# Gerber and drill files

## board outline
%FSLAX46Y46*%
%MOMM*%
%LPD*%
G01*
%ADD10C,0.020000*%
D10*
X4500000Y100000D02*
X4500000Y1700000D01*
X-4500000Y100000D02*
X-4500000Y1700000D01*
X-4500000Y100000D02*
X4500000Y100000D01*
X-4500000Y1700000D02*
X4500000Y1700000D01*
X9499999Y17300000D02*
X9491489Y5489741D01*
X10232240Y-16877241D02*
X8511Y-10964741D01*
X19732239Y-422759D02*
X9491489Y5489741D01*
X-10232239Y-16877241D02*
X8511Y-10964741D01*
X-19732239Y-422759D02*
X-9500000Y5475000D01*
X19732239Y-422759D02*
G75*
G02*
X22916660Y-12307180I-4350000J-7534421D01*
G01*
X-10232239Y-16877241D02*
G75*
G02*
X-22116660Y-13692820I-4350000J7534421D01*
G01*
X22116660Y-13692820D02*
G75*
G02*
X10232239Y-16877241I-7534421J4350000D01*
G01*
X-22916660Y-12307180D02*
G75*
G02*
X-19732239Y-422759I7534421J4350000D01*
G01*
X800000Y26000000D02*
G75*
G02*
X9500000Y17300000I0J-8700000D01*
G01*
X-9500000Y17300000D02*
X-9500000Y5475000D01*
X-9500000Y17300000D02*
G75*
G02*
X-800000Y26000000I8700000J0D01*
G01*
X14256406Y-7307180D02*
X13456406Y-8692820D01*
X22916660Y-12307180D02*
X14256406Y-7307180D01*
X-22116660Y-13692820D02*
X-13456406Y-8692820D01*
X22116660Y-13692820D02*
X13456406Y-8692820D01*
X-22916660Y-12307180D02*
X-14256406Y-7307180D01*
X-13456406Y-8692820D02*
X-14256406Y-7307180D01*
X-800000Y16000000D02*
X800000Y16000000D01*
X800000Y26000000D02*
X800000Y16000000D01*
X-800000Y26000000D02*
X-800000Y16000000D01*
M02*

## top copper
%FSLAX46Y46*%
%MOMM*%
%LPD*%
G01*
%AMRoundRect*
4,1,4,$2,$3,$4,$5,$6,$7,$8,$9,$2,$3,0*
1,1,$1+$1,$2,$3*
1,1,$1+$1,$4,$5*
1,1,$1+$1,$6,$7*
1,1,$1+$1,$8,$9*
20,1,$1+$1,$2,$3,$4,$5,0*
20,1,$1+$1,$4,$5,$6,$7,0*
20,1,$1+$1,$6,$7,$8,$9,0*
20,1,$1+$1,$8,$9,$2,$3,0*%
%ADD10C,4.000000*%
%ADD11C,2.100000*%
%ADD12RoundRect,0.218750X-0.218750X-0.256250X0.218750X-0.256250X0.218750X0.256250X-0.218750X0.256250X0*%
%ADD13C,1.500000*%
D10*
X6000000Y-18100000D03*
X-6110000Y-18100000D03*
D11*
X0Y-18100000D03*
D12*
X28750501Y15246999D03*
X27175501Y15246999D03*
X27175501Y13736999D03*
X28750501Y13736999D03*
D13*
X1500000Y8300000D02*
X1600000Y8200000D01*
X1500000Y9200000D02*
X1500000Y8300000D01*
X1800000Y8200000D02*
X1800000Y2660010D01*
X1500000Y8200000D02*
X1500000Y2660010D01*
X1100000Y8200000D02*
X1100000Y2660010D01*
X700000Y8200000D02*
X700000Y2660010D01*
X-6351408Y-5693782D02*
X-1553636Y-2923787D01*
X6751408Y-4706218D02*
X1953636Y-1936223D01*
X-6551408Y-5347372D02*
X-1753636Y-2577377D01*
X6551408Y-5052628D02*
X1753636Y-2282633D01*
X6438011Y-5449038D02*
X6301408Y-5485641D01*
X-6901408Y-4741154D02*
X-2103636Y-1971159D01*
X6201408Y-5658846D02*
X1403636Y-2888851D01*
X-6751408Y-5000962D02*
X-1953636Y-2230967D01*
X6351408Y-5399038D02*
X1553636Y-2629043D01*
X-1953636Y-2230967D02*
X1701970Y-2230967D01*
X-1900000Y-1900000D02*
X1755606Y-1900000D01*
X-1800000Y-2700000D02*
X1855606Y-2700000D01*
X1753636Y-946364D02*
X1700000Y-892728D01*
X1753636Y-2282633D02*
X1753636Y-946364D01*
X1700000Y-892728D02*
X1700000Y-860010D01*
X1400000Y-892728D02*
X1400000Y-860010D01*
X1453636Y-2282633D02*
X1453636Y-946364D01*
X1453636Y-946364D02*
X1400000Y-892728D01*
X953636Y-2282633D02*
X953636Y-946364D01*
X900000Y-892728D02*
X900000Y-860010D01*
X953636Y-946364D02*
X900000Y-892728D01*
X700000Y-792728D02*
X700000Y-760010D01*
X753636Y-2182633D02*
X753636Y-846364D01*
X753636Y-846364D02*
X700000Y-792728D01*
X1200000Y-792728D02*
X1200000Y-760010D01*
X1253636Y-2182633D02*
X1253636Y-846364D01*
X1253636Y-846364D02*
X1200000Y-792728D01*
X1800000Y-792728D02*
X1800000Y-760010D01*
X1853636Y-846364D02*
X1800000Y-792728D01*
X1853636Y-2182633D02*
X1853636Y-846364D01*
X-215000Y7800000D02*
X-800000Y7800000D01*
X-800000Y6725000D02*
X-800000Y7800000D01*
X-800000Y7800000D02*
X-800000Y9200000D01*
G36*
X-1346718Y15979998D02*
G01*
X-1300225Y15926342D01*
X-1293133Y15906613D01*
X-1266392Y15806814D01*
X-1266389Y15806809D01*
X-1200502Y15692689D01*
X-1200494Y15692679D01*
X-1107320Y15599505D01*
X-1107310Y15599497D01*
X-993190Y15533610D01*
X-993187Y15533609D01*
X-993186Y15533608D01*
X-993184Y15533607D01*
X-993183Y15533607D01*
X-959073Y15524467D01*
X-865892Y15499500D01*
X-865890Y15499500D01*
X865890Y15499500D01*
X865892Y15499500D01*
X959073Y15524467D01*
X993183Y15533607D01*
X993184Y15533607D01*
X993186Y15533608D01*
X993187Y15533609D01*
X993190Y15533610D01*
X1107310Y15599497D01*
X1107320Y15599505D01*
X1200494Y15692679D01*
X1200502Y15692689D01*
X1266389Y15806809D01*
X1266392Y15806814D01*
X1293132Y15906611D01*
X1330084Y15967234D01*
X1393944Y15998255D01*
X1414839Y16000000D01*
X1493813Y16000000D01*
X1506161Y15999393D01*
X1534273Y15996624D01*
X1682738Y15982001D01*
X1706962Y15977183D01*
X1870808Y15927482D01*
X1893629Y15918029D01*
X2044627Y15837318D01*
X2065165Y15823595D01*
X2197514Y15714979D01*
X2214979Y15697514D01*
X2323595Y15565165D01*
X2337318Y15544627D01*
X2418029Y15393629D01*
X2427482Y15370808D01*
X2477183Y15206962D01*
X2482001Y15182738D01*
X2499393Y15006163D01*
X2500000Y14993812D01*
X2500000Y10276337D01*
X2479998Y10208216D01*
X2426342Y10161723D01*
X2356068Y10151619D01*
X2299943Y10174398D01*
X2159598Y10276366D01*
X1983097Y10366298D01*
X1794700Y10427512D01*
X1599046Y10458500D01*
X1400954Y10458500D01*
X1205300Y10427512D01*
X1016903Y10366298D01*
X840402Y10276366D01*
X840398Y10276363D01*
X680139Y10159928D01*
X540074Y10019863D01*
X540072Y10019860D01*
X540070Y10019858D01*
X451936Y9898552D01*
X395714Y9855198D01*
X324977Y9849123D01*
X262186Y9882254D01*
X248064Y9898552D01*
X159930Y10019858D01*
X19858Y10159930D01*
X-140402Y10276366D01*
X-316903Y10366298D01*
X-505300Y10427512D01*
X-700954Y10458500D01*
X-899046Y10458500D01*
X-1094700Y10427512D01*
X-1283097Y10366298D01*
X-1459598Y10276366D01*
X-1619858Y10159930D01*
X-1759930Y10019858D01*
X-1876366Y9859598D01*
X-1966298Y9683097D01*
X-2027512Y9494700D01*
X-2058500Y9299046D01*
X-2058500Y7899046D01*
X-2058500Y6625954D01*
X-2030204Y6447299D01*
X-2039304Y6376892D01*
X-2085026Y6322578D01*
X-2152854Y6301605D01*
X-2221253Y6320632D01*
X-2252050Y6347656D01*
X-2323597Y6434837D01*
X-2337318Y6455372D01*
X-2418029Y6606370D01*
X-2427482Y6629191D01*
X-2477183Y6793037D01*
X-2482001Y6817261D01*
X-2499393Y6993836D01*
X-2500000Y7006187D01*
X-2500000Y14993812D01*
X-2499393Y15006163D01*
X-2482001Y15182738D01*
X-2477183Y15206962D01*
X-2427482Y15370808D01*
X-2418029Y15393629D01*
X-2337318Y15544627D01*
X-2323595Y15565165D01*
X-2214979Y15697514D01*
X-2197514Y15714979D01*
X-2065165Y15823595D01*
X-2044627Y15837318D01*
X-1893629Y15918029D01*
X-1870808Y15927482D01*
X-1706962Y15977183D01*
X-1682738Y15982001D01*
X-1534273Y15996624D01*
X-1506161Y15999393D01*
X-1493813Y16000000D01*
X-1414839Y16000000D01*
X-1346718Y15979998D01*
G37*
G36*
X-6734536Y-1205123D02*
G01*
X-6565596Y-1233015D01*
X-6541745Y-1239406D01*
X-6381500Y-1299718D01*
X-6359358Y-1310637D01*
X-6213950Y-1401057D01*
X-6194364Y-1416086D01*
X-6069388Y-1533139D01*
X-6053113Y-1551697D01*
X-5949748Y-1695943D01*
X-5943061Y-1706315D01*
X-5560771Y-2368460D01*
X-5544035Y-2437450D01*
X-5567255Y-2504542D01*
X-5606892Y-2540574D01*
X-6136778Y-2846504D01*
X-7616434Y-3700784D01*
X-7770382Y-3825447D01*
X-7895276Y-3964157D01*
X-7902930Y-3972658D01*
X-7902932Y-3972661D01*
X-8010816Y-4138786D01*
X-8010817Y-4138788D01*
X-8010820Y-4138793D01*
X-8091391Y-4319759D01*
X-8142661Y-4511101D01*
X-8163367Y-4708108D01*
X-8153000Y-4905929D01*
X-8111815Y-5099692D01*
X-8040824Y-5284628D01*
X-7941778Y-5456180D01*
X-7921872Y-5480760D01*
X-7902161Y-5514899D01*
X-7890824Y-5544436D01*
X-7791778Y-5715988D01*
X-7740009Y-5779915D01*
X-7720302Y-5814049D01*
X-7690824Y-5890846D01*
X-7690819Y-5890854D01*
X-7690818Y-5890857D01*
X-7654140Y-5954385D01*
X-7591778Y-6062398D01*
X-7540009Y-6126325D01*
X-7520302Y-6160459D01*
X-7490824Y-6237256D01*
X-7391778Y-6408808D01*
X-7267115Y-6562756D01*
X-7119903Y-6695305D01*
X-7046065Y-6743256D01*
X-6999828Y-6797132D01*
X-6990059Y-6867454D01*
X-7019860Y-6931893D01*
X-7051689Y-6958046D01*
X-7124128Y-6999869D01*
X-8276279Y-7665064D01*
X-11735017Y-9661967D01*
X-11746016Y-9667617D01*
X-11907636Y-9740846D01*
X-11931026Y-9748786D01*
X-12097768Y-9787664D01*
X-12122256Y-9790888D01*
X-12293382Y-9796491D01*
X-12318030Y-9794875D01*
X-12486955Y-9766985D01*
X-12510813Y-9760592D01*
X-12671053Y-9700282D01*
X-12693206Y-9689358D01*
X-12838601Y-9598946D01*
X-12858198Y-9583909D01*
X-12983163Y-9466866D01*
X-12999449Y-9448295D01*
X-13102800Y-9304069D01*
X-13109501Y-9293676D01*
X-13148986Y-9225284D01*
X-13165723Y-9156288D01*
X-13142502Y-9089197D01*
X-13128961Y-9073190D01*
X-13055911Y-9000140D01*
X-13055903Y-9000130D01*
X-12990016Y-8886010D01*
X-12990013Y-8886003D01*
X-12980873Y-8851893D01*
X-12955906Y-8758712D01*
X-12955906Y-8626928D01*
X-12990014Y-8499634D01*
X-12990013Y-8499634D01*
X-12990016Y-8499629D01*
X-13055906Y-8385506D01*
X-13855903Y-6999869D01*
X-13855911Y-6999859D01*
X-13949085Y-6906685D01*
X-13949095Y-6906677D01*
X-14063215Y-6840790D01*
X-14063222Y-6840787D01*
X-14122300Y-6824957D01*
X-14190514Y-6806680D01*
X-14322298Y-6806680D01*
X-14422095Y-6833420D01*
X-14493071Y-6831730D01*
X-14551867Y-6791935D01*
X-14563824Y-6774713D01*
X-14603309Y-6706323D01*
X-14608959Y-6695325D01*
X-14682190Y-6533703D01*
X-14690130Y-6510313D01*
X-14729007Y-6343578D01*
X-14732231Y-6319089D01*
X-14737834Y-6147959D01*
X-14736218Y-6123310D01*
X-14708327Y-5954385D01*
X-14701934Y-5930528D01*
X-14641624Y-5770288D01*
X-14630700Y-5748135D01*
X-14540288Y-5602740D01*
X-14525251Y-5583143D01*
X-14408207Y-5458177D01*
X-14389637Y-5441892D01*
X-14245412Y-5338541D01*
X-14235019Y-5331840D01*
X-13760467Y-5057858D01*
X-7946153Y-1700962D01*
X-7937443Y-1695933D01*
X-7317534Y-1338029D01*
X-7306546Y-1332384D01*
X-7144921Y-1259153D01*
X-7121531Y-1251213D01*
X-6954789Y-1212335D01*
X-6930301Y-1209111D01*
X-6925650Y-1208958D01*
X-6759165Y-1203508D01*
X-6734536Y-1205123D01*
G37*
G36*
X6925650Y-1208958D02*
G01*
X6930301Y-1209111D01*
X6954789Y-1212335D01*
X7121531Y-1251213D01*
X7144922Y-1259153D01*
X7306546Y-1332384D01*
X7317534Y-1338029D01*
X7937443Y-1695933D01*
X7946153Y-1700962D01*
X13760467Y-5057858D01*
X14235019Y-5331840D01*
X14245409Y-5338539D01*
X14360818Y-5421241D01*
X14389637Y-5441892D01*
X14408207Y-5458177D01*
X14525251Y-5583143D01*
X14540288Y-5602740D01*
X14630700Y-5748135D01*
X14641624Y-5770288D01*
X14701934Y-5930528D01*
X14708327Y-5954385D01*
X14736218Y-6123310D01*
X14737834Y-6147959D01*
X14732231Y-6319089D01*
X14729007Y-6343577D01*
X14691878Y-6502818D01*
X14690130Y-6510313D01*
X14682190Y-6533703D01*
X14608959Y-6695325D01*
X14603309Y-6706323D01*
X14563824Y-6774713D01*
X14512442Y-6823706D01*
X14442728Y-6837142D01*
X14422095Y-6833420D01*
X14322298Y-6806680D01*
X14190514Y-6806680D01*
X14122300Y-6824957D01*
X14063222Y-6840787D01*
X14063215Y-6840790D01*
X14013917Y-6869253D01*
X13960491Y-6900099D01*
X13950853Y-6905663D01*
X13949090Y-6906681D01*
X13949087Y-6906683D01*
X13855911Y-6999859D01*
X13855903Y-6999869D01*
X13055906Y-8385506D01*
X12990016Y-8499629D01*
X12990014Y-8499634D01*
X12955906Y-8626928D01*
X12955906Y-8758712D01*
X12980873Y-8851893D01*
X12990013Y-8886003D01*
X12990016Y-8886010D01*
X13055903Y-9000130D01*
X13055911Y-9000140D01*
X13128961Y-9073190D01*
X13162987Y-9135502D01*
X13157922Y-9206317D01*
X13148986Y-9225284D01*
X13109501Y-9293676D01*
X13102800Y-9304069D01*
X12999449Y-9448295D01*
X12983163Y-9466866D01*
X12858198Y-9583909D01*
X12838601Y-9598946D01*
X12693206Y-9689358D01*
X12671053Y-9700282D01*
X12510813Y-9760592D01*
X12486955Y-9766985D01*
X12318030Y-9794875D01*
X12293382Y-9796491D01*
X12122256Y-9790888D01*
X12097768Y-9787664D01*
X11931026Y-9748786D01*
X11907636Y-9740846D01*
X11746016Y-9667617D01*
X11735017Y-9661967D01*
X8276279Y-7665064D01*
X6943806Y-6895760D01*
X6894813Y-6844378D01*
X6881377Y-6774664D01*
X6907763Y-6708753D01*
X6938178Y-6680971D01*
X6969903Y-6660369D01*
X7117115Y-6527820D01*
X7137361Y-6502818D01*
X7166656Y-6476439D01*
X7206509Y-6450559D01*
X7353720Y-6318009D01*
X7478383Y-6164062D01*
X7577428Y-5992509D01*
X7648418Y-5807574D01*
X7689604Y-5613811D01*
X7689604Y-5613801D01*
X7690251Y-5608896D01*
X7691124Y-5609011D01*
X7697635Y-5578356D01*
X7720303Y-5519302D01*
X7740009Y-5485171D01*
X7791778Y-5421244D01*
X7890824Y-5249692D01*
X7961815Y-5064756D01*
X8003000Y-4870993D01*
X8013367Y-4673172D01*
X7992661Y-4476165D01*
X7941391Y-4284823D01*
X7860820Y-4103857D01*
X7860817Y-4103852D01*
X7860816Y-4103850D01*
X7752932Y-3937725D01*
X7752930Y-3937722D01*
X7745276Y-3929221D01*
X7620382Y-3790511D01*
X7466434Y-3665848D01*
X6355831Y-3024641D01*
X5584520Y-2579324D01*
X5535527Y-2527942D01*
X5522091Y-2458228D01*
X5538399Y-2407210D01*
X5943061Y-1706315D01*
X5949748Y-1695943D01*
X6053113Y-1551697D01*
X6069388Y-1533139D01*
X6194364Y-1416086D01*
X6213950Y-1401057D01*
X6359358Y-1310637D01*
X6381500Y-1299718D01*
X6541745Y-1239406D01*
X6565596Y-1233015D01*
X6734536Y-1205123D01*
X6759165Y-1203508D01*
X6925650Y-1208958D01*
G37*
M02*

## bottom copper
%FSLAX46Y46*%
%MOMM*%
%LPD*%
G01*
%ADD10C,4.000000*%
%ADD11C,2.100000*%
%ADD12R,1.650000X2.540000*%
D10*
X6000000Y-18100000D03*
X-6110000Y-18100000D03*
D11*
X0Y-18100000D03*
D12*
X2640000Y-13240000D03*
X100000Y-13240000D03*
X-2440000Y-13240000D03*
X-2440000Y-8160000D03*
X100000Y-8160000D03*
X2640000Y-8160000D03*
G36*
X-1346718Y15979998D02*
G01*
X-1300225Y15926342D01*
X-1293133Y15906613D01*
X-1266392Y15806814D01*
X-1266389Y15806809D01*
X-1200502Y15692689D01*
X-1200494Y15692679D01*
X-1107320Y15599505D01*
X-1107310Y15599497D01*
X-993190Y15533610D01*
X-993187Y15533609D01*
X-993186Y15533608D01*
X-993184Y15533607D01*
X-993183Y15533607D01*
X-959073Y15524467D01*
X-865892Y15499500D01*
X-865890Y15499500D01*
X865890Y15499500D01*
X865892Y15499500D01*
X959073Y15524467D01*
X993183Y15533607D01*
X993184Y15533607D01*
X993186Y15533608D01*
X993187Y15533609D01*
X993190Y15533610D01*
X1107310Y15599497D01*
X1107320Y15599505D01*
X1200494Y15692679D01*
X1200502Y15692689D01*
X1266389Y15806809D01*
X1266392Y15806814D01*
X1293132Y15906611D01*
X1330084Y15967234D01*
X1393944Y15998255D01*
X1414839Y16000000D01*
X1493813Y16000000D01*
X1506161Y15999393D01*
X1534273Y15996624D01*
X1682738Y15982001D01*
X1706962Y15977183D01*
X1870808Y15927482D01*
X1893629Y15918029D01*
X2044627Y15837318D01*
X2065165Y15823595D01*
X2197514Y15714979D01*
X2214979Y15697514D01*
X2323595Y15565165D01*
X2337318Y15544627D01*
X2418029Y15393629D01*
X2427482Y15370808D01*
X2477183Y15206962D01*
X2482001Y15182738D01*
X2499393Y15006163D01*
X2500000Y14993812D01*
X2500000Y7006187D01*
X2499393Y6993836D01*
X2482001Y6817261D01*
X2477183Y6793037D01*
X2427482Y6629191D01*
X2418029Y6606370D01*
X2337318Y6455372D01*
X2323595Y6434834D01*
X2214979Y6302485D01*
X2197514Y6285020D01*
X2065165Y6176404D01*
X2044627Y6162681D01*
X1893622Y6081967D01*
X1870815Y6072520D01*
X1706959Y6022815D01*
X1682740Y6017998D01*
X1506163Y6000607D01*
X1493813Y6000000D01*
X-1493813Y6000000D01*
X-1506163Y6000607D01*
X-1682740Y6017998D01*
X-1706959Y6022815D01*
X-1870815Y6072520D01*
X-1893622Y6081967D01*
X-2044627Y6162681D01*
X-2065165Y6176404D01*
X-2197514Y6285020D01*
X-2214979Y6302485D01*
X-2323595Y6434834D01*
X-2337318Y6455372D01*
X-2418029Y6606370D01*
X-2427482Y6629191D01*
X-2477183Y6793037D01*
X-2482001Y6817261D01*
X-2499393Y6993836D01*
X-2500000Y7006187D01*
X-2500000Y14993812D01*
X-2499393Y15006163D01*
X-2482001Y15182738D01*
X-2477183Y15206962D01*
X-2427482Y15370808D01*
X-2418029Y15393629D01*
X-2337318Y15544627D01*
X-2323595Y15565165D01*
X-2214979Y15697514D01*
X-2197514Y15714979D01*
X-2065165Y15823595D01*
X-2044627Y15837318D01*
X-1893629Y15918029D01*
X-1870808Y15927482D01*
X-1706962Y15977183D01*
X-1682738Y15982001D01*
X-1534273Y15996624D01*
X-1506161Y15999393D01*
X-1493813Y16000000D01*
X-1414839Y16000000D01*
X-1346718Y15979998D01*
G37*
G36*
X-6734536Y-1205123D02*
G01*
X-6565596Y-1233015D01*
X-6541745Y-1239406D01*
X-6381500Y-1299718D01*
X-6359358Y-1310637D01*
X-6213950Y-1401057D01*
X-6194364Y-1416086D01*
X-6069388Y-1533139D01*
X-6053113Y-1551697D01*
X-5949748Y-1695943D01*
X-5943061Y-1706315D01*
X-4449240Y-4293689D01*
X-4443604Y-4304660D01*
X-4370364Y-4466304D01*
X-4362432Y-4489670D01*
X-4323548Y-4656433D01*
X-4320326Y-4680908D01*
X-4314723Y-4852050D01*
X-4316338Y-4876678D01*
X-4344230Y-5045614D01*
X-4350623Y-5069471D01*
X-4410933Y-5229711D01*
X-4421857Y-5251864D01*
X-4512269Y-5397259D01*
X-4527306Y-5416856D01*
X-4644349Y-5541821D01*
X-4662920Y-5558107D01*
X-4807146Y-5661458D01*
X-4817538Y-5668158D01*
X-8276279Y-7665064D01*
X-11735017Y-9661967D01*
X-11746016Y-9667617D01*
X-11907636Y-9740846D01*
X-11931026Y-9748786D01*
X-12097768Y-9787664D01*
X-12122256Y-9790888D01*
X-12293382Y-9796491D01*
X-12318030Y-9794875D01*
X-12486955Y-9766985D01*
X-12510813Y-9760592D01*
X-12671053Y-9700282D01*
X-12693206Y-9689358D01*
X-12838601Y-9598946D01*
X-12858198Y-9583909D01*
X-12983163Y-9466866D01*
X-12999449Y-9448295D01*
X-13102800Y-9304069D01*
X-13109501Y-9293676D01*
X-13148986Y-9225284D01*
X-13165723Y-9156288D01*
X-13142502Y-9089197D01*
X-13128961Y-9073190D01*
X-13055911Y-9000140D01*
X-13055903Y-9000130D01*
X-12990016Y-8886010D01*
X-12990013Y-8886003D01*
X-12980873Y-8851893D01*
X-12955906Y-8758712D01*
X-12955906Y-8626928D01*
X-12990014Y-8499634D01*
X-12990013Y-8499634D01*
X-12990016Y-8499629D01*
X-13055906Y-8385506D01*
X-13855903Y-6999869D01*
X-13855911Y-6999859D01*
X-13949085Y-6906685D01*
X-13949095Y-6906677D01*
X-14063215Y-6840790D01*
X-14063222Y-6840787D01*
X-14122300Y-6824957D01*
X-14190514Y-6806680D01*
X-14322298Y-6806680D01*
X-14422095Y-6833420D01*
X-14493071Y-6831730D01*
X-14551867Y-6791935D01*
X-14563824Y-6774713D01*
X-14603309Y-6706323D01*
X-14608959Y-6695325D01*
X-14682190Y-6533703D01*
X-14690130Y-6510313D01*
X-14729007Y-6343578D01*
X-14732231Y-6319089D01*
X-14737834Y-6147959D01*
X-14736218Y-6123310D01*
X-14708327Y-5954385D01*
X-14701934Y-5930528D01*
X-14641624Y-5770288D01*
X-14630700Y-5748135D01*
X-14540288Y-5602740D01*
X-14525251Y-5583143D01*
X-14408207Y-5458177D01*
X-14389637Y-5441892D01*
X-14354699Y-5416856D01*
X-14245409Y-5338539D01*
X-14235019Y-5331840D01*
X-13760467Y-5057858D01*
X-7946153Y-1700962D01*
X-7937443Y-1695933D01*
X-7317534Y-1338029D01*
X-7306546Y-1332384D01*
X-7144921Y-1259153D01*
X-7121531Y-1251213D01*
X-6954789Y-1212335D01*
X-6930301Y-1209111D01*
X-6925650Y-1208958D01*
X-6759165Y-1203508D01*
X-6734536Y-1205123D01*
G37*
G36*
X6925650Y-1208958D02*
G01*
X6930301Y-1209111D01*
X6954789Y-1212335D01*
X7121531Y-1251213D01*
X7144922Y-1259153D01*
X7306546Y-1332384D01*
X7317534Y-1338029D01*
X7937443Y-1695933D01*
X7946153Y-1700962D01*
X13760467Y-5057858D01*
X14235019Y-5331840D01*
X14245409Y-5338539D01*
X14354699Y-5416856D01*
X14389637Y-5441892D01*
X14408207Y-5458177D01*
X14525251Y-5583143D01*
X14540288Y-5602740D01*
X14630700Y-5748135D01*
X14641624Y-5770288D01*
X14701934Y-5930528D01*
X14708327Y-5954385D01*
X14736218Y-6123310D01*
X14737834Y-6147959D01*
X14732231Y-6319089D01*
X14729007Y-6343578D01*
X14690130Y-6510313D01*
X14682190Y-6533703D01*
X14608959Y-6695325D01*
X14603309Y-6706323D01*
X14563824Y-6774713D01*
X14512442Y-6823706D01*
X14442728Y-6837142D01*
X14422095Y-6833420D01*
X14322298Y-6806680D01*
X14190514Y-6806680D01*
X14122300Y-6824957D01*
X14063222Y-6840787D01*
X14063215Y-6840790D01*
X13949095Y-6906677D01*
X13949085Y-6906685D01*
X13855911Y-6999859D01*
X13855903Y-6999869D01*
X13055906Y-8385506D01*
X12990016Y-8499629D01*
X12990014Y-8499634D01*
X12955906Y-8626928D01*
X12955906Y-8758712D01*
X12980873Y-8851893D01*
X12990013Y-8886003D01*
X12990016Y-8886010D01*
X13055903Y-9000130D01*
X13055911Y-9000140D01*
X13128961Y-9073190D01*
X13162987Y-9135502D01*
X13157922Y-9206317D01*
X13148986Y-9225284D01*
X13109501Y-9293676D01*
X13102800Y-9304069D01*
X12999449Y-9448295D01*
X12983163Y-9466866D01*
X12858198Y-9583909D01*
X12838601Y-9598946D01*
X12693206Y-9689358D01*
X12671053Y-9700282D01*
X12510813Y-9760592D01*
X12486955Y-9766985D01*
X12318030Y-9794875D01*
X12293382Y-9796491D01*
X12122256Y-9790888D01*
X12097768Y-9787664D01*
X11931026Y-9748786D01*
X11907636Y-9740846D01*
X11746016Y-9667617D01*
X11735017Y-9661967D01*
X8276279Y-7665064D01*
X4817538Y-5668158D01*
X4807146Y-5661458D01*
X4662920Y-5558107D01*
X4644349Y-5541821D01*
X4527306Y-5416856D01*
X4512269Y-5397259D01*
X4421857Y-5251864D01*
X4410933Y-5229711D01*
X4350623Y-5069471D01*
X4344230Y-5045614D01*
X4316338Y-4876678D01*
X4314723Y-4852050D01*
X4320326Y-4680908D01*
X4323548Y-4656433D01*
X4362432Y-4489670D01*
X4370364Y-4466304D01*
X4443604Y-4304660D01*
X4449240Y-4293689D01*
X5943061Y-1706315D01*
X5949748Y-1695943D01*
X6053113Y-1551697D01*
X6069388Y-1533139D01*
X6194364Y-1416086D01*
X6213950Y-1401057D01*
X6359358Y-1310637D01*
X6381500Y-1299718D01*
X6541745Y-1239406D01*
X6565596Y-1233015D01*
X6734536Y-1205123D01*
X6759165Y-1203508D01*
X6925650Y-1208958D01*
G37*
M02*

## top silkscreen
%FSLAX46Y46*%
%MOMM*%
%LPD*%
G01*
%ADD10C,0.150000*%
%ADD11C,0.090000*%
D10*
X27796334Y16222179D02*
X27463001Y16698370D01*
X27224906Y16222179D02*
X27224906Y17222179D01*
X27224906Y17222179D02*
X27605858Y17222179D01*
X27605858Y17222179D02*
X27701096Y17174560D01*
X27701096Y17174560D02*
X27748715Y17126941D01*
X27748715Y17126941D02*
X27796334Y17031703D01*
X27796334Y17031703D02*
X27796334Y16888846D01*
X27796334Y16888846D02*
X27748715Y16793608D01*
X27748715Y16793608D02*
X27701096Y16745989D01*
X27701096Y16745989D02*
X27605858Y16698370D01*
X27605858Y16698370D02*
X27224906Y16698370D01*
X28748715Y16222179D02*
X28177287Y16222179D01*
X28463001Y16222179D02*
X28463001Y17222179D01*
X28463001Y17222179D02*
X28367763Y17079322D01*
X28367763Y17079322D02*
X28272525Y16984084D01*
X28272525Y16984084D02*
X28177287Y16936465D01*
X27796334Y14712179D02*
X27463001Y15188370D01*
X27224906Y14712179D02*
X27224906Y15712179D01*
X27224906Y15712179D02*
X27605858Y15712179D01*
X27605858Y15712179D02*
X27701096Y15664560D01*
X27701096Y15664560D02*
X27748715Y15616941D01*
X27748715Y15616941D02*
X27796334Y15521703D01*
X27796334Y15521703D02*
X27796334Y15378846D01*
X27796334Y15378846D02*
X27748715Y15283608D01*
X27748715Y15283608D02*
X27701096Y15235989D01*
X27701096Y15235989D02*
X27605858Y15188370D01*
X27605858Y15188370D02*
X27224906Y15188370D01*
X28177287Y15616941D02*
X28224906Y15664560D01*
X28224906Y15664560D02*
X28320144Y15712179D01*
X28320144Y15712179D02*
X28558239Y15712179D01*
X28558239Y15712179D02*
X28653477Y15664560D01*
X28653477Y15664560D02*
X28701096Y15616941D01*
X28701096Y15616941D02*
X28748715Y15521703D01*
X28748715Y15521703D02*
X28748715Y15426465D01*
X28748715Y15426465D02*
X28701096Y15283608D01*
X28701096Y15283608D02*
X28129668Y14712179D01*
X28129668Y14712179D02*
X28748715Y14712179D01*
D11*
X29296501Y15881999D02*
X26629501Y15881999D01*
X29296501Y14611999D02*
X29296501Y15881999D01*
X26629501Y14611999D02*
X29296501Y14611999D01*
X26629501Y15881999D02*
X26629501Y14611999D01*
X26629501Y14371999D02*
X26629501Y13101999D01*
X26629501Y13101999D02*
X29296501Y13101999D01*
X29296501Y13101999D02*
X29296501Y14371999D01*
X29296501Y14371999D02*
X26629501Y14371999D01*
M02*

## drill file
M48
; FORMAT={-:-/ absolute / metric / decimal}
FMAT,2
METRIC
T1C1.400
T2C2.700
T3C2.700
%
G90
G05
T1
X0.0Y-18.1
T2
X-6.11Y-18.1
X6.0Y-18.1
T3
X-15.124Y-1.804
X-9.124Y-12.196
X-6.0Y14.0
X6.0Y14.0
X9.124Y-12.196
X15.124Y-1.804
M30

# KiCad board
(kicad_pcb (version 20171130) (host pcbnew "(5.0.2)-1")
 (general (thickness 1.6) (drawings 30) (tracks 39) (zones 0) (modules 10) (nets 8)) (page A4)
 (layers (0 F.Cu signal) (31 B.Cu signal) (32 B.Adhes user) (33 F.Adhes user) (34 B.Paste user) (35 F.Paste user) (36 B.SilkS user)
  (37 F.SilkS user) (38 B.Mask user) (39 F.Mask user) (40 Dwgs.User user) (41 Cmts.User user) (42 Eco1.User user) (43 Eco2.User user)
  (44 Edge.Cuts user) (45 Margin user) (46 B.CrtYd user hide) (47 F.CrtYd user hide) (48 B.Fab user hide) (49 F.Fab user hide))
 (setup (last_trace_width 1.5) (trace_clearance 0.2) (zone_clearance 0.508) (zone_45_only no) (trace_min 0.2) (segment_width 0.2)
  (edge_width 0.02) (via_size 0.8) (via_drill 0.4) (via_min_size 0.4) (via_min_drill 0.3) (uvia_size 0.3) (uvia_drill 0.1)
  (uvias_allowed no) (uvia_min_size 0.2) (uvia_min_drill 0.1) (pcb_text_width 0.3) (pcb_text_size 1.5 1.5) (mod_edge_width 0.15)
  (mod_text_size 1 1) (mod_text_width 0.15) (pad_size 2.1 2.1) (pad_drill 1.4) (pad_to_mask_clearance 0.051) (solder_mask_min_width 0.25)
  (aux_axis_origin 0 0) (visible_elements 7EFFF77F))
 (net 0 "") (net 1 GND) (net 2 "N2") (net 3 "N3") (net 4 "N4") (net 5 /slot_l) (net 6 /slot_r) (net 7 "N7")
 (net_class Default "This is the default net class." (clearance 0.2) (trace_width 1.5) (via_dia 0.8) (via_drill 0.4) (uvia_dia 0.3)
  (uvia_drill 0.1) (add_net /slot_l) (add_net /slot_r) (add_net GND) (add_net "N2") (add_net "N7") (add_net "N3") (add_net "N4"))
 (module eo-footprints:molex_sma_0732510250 (layer F.Cu) (at 0 18.1 180)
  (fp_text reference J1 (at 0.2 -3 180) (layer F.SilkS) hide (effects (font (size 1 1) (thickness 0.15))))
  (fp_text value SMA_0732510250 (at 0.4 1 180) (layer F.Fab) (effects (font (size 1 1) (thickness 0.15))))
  (pad 2 thru_hole circle (at -6 0 180) (size 4 4) (drill 2.7) (layers *.Cu *.Mask) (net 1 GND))
  (pad 2 thru_hole circle (at 6.11 0 180) (size 4 4) (drill 2.7) (layers *.Cu *.Mask) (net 1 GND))
  (pad 1 thru_hole circle (at 0 0 180) (size 2.1 2.1) (drill 1.4) (layers *.Cu *.Mask) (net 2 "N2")))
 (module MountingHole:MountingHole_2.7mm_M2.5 (layer F.Cu) (at 15.124356 1.803848 240)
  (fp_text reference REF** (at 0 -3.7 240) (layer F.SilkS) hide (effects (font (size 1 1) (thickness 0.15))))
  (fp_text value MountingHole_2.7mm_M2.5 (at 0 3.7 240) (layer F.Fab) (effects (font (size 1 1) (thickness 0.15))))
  (pad 1 np_thru_hole circle (at 0 0 240) (size 2.7 2.7) (drill 2.7) (layers *.Cu *.Mask)))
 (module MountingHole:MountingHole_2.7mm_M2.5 (layer F.Cu) (at -9.124356 12.196152 120)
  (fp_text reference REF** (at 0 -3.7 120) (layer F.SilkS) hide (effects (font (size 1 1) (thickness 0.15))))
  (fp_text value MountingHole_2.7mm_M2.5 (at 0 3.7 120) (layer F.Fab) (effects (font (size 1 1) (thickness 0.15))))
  (pad 1 np_thru_hole circle (at 0 0 120) (size 2.7 2.7) (drill 2.7) (layers *.Cu *.Mask)))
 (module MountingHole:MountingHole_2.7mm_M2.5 (layer F.Cu) (at 9.124356 12.196152 240)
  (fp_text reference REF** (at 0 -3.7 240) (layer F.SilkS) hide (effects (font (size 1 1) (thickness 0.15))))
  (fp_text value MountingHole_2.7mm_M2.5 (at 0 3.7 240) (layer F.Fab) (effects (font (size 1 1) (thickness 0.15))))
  (pad 1 np_thru_hole circle (at 0 0 240) (size 2.7 2.7) (drill 2.7) (layers *.Cu *.Mask)))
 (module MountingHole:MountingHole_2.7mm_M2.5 (layer F.Cu) (at -15.124356 1.803848 120)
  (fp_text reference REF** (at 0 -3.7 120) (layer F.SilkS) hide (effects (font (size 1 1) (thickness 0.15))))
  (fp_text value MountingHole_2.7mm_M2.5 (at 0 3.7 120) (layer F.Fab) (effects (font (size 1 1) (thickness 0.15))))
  (pad 1 np_thru_hole circle (at 0 0 120) (size 2.7 2.7) (drill 2.7) (layers *.Cu *.Mask)))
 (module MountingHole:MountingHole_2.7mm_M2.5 (layer F.Cu) (at 6 -14)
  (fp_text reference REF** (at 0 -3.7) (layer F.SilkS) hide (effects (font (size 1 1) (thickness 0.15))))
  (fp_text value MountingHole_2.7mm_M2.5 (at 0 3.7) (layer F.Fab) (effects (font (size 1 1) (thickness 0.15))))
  (pad 1 np_thru_hole circle (at 0 0) (size 2.7 2.7) (drill 2.7) (layers *.Cu *.Mask)))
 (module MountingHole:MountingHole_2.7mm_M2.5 (layer F.Cu) (at -6 -14)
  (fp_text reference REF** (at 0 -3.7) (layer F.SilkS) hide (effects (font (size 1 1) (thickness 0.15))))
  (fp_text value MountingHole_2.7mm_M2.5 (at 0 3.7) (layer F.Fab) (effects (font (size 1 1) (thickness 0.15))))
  (pad 1 np_thru_hole circle (at 0 0) (size 2.7 2.7) (drill 2.7) (layers *.Cu *.Mask)))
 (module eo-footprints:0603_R (layer F.Cu) (at 27.963001 -15.246999)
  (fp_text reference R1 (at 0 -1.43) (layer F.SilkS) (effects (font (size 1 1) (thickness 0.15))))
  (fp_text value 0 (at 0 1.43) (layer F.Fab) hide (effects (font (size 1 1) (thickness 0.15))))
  (fp_line (start 1.3335 -0.635) (end -1.3335 -0.635) (layer F.SilkS) (width 0.09))
  (fp_line (start 1.3335 0.635) (end 1.3335 -0.635) (layer F.SilkS) (width 0.09))
  (fp_line (start -1.3335 0.635) (end 1.3335 0.635) (layer F.SilkS) (width 0.09))
  (fp_line (start -1.3335 -0.635) (end -1.3335 0.635) (layer F.SilkS) (width 0.09))
  (pad 2 smd roundrect (at 0.7875 0) (size 0.875 0.95) (layers F.Cu F.Paste F.Mask) (roundrect_rratio 0.25) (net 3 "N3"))
  (pad 1 smd roundrect (at -0.7875 0) (size 0.875 0.95) (layers F.Cu F.Paste F.Mask) (roundrect_rratio 0.25) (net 1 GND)))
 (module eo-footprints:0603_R (layer F.Cu) (at 27.963001 -13.736999)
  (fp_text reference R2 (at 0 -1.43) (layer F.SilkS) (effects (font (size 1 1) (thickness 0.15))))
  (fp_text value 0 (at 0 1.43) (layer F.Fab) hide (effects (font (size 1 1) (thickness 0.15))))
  (fp_line (start -1.3335 -0.635) (end -1.3335 0.635) (layer F.SilkS) (width 0.09))
  (fp_line (start -1.3335 0.635) (end 1.3335 0.635) (layer F.SilkS) (width 0.09))
  (fp_line (start 1.3335 0.635) (end 1.3335 -0.635) (layer F.SilkS) (width 0.09))
  (fp_line (start 1.3335 -0.635) (end -1.3335 -0.635) (layer F.SilkS) (width 0.09))
  (pad 1 smd roundrect (at -0.7875 0) (size 0.875 0.95) (layers F.Cu F.Paste F.Mask) (roundrect_rratio 0.25) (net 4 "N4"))
  (pad 2 smd roundrect (at 0.7875 0) (size 0.875 0.95) (layers F.Cu F.Paste F.Mask) (roundrect_rratio 0.25) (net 1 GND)))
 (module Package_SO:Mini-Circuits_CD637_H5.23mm (layer B.Cu) (at 0.1 10.7 90)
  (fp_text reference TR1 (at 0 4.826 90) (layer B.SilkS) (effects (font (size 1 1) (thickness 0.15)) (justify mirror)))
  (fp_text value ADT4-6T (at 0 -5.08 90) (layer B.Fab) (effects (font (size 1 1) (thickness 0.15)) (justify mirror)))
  (pad 1 smd rect (at -2.54 2.54 90) (size 2.54 1.65) (layers B.Cu B.Paste B.Mask) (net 4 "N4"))
  (pad 2 smd rect (at -2.54 0 90) (size 2.54 1.65) (layers B.Cu B.Paste B.Mask))
  (pad 3 smd rect (at -2.54 -2.54 90) (size 2.54 1.65) (layers B.Cu B.Paste B.Mask) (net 2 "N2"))
  (pad 4 smd rect (at 2.54 -2.54 90) (size 2.54 1.65) (layers B.Cu B.Paste B.Mask) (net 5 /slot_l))
  (pad 5 smd rect (at 2.54 0 90) (size 2.54 1.65) (layers B.Cu B.Paste B.Mask) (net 3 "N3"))
  (pad 6 smd rect (at 2.54 2.54 90) (size 2.54 1.65) (layers B.Cu B.Paste B.Mask) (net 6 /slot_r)))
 (gr_line (start 4.5 -0.1) (end 4.5 -1.7) (layer Edge.Cuts) (width 0.02))
 (gr_line (start -4.5 -0.1) (end -4.5 -1.7) (layer Edge.Cuts) (width 0.02))
 (gr_line (start -4.5 -0.1) (end 4.5 -0.1) (layer Edge.Cuts) (width 0.02))
 (gr_line (start -4.5 -1.7) (end 4.5 -1.7) (layer Edge.Cuts) (width 0.02))
 (gr_line (start 9.499999 -17.3) (end 9.491489 -5.489741) (layer Edge.Cuts) (width 0.02))
 (gr_line (start 10.23224 16.877241) (end 0.008511 10.964741) (layer Edge.Cuts) (width 0.02))
 (gr_line (start 19.732239 0.422759) (end 9.491489 -5.489741) (layer Edge.Cuts) (width 0.02))
 (gr_line (start -10.232239 16.877241) (end 0.008511 10.964741) (layer Edge.Cuts) (width 0.02))
 (gr_line (start -19.732239 0.422759) (end -9.5 -5.475) (layer Edge.Cuts) (width 0.02))
 (gr_arc (start 15.382239 7.95718) (end 22.91666 12.30718) (angle -90) (layer Edge.Cuts) (width 0.02))
 (gr_arc (start -14.582239 9.34282) (end -22.11666 13.69282) (angle -90) (layer Edge.Cuts) (width 0.02))
 (gr_arc (start 14.582239 9.34282) (end 10.232239 16.877241) (angle -90) (layer Edge.Cuts) (width 0.02))
 (gr_arc (start -15.382239 7.95718) (end -19.732239 0.422759) (angle -90) (layer Edge.Cuts) (width 0.02))
 (gr_arc (start 0.8 -17.3) (end 9.5 -17.3) (angle -90) (layer Edge.Cuts) (width 0.02))
 (gr_line (start -9.5 -17.3) (end -9.5 -5.475) (layer Edge.Cuts) (width 0.02))
 (gr_arc (start -0.8 -17.3) (end -0.8 -26) (angle -90) (layer Edge.Cuts) (width 0.02))
 (gr_line (start 14.256406 7.30718) (end 13.456406 8.69282) (layer Edge.Cuts) (width 0.02))
 (gr_line (start 22.91666 12.30718) (end 14.256406 7.30718) (layer Edge.Cuts) (width 0.02))
 (gr_line (start -22.11666 13.69282) (end -13.456406 8.69282) (layer Edge.Cuts) (width 0.02))
 (gr_line (start 22.11666 13.69282) (end 13.456406 8.69282) (layer Edge.Cuts) (width 0.02))
 (gr_line (start -22.91666 12.30718) (end -14.256406 7.30718) (layer Edge.Cuts) (width 0.02))
 (gr_line (start -13.456406 8.69282) (end -14.256406 7.30718) (layer Edge.Cuts) (width 0.02))
 (gr_line (start -0.8 -16) (end 0.8 -16) (layer Edge.Cuts) (width 0.02))
 (gr_line (start 0.8 -26) (end 0.8 -16) (layer Edge.Cuts) (width 0.02))
 (gr_line (start -0.8 -26) (end -0.8 -16) (layer Edge.Cuts) (width 0.02))
 (segment (start 1.5 -8.3) (end 1.6 -8.2) (width 1.5) (layer F.Cu) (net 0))
 (segment (start 1.5 -9.2) (end 1.5 -8.3) (width 1.5) (layer F.Cu) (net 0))
 (segment (start 1.8 -8.2) (end 1.8 -2.66001) (width 1.5) (layer F.Cu) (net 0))
 (segment (start 1.5 -8.2) (end 1.5 -2.66001) (width 1.5) (layer F.Cu) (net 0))
 (segment (start 1.1 -8.2) (end 1.1 -2.66001) (width 1.5) (layer F.Cu) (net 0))
 (segment (start 0.7 -8.2) (end 0.7 -2.66001) (width 1.5) (layer F.Cu) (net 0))
 (segment (start -6.351408 5.693782) (end -1.553636 2.923787) (width 1.5) (layer F.Cu) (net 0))
 (segment (start 6.751408 4.706218) (end 1.953636 1.936223) (width 1.5) (layer F.Cu) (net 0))
 (segment (start -6.551408 5.347372) (end -1.753636 2.577377) (width 1.5) (layer F.Cu) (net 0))
 (segment (start 6.551408 5.052628) (end 1.753636 2.282633) (width 1.5) (layer F.Cu) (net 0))
 (segment (start 6.438011 5.449038) (end 6.301408 5.485641) (width 1.5) (layer F.Cu) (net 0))
 (segment (start -6.901408 4.741154) (end -2.103636 1.971159) (width 1.5) (layer F.Cu) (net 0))
 (segment (start 6.201408 5.658846) (end 1.403636 2.888851) (width 1.5) (layer F.Cu) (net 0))
 (segment (start -6.751408 5.000962) (end -1.953636 2.230967) (width 1.5) (layer F.Cu) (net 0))
 (segment (start 6.351408 5.399038) (end 1.553636 2.629043) (width 1.5) (layer F.Cu) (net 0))
 (segment (start -1.953636 2.230967) (end 1.70197 2.230967) (width 1.5) (layer F.Cu) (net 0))
 (segment (start -1.9 1.9) (end 1.755606 1.9) (width 1.5) (layer F.Cu) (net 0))
 (segment (start -1.8 2.7) (end 1.855606 2.7) (width 1.5) (layer F.Cu) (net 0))
 (segment (start 1.753636 0.946364) (end 1.7 0.892728) (width 1.5) (layer F.Cu) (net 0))
 (segment (start 1.753636 2.282633) (end 1.753636 0.946364) (width 1.5) (layer F.Cu) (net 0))
 (segment (start 1.7 0.892728) (end 1.7 0.86001) (width 1.5) (layer F.Cu) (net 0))
 (segment (start 1.4 0.892728) (end 1.4 0.86001) (width 1.5) (layer F.Cu) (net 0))
 (segment (start 1.453636 2.282633) (end 1.453636 0.946364) (width 1.5) (layer F.Cu) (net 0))
 (segment (start 1.453636 0.946364) (end 1.4 0.892728) (width 1.5) (layer F.Cu) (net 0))
 (segment (start 0.953636 2.282633) (end 0.953636 0.946364) (width 1.5) (layer F.Cu) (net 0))
 (segment (start 0.9 0.892728) (end 0.9 0.86001) (width 1.5) (layer F.Cu) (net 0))
 (segment (start 0.953636 0.946364) (end 0.9 0.892728) (width 1.5) (layer F.Cu) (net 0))
 (segment (start 0.7 0.792728) (end 0.7 0.76001) (width 1.5) (layer F.Cu) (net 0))
 (segment (start 0.753636 2.182633) (end 0.753636 0.846364) (width 1.5) (layer F.Cu) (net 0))
 (segment (start 0.753636 0.846364) (end 0.7 0.792728) (width 1.5) (layer F.Cu) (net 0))
 (segment (start 1.2 0.792728) (end 1.2 0.76001) (width 1.5) (layer F.Cu) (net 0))
 (segment (start 1.253636 2.182633) (end 1.253636 0.846364) (width 1.5) (layer F.Cu) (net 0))
 (segment (start 1.253636 0.846364) (end 1.2 0.792728) (width 1.5) (layer F.Cu) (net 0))
 (segment (start 1.8 0.792728) (end 1.8 0.76001) (width 1.5) (layer F.Cu) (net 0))
 (segment (start 1.853636 0.846364) (end 1.8 0.792728) (width 1.5) (layer F.Cu) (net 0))
 (segment (start 1.853636 2.182633) (end 1.853636 0.846364) (width 1.5) (layer F.Cu) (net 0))
 (segment (start -0.215 -7.8) (end -0.8 -7.8) (width 1.5) (layer F.Cu) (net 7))
 (segment (start -0.8 -6.725) (end -0.8 -7.8) (width 1.5) (layer F.Cu) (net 7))
 (segment (start -0.8 -7.8) (end -0.8 -9.2) (width 1.5) (layer F.Cu) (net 7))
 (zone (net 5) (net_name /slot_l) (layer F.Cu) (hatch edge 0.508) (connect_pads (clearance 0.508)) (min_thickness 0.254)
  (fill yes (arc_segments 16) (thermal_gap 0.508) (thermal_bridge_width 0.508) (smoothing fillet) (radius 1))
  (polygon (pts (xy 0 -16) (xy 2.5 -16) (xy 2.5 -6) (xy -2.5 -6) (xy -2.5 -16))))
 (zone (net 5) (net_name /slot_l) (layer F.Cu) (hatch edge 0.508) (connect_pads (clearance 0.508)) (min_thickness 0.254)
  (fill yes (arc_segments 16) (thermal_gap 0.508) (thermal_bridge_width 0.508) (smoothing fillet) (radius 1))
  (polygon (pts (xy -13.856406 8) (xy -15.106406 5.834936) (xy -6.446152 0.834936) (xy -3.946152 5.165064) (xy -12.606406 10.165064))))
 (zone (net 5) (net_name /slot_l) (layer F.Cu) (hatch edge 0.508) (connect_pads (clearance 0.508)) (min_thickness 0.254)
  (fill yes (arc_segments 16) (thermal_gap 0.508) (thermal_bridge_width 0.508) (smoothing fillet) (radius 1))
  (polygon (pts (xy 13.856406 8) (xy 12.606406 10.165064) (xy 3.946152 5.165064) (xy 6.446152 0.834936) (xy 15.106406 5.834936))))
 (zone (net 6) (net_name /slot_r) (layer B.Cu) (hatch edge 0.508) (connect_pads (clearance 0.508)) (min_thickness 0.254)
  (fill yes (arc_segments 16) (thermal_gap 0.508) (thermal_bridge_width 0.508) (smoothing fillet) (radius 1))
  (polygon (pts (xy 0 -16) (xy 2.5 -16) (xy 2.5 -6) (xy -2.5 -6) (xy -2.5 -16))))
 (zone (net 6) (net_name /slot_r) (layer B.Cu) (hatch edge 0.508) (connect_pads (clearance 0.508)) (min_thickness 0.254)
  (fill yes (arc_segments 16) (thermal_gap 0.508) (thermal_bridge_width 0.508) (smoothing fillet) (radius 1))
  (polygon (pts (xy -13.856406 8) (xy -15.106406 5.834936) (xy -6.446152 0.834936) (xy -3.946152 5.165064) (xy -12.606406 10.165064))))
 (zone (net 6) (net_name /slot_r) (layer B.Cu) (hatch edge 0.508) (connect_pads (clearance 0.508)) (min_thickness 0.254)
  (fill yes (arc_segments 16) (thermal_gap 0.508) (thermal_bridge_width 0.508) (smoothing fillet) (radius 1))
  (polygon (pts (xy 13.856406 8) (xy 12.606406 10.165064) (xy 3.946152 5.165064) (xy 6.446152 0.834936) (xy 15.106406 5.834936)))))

